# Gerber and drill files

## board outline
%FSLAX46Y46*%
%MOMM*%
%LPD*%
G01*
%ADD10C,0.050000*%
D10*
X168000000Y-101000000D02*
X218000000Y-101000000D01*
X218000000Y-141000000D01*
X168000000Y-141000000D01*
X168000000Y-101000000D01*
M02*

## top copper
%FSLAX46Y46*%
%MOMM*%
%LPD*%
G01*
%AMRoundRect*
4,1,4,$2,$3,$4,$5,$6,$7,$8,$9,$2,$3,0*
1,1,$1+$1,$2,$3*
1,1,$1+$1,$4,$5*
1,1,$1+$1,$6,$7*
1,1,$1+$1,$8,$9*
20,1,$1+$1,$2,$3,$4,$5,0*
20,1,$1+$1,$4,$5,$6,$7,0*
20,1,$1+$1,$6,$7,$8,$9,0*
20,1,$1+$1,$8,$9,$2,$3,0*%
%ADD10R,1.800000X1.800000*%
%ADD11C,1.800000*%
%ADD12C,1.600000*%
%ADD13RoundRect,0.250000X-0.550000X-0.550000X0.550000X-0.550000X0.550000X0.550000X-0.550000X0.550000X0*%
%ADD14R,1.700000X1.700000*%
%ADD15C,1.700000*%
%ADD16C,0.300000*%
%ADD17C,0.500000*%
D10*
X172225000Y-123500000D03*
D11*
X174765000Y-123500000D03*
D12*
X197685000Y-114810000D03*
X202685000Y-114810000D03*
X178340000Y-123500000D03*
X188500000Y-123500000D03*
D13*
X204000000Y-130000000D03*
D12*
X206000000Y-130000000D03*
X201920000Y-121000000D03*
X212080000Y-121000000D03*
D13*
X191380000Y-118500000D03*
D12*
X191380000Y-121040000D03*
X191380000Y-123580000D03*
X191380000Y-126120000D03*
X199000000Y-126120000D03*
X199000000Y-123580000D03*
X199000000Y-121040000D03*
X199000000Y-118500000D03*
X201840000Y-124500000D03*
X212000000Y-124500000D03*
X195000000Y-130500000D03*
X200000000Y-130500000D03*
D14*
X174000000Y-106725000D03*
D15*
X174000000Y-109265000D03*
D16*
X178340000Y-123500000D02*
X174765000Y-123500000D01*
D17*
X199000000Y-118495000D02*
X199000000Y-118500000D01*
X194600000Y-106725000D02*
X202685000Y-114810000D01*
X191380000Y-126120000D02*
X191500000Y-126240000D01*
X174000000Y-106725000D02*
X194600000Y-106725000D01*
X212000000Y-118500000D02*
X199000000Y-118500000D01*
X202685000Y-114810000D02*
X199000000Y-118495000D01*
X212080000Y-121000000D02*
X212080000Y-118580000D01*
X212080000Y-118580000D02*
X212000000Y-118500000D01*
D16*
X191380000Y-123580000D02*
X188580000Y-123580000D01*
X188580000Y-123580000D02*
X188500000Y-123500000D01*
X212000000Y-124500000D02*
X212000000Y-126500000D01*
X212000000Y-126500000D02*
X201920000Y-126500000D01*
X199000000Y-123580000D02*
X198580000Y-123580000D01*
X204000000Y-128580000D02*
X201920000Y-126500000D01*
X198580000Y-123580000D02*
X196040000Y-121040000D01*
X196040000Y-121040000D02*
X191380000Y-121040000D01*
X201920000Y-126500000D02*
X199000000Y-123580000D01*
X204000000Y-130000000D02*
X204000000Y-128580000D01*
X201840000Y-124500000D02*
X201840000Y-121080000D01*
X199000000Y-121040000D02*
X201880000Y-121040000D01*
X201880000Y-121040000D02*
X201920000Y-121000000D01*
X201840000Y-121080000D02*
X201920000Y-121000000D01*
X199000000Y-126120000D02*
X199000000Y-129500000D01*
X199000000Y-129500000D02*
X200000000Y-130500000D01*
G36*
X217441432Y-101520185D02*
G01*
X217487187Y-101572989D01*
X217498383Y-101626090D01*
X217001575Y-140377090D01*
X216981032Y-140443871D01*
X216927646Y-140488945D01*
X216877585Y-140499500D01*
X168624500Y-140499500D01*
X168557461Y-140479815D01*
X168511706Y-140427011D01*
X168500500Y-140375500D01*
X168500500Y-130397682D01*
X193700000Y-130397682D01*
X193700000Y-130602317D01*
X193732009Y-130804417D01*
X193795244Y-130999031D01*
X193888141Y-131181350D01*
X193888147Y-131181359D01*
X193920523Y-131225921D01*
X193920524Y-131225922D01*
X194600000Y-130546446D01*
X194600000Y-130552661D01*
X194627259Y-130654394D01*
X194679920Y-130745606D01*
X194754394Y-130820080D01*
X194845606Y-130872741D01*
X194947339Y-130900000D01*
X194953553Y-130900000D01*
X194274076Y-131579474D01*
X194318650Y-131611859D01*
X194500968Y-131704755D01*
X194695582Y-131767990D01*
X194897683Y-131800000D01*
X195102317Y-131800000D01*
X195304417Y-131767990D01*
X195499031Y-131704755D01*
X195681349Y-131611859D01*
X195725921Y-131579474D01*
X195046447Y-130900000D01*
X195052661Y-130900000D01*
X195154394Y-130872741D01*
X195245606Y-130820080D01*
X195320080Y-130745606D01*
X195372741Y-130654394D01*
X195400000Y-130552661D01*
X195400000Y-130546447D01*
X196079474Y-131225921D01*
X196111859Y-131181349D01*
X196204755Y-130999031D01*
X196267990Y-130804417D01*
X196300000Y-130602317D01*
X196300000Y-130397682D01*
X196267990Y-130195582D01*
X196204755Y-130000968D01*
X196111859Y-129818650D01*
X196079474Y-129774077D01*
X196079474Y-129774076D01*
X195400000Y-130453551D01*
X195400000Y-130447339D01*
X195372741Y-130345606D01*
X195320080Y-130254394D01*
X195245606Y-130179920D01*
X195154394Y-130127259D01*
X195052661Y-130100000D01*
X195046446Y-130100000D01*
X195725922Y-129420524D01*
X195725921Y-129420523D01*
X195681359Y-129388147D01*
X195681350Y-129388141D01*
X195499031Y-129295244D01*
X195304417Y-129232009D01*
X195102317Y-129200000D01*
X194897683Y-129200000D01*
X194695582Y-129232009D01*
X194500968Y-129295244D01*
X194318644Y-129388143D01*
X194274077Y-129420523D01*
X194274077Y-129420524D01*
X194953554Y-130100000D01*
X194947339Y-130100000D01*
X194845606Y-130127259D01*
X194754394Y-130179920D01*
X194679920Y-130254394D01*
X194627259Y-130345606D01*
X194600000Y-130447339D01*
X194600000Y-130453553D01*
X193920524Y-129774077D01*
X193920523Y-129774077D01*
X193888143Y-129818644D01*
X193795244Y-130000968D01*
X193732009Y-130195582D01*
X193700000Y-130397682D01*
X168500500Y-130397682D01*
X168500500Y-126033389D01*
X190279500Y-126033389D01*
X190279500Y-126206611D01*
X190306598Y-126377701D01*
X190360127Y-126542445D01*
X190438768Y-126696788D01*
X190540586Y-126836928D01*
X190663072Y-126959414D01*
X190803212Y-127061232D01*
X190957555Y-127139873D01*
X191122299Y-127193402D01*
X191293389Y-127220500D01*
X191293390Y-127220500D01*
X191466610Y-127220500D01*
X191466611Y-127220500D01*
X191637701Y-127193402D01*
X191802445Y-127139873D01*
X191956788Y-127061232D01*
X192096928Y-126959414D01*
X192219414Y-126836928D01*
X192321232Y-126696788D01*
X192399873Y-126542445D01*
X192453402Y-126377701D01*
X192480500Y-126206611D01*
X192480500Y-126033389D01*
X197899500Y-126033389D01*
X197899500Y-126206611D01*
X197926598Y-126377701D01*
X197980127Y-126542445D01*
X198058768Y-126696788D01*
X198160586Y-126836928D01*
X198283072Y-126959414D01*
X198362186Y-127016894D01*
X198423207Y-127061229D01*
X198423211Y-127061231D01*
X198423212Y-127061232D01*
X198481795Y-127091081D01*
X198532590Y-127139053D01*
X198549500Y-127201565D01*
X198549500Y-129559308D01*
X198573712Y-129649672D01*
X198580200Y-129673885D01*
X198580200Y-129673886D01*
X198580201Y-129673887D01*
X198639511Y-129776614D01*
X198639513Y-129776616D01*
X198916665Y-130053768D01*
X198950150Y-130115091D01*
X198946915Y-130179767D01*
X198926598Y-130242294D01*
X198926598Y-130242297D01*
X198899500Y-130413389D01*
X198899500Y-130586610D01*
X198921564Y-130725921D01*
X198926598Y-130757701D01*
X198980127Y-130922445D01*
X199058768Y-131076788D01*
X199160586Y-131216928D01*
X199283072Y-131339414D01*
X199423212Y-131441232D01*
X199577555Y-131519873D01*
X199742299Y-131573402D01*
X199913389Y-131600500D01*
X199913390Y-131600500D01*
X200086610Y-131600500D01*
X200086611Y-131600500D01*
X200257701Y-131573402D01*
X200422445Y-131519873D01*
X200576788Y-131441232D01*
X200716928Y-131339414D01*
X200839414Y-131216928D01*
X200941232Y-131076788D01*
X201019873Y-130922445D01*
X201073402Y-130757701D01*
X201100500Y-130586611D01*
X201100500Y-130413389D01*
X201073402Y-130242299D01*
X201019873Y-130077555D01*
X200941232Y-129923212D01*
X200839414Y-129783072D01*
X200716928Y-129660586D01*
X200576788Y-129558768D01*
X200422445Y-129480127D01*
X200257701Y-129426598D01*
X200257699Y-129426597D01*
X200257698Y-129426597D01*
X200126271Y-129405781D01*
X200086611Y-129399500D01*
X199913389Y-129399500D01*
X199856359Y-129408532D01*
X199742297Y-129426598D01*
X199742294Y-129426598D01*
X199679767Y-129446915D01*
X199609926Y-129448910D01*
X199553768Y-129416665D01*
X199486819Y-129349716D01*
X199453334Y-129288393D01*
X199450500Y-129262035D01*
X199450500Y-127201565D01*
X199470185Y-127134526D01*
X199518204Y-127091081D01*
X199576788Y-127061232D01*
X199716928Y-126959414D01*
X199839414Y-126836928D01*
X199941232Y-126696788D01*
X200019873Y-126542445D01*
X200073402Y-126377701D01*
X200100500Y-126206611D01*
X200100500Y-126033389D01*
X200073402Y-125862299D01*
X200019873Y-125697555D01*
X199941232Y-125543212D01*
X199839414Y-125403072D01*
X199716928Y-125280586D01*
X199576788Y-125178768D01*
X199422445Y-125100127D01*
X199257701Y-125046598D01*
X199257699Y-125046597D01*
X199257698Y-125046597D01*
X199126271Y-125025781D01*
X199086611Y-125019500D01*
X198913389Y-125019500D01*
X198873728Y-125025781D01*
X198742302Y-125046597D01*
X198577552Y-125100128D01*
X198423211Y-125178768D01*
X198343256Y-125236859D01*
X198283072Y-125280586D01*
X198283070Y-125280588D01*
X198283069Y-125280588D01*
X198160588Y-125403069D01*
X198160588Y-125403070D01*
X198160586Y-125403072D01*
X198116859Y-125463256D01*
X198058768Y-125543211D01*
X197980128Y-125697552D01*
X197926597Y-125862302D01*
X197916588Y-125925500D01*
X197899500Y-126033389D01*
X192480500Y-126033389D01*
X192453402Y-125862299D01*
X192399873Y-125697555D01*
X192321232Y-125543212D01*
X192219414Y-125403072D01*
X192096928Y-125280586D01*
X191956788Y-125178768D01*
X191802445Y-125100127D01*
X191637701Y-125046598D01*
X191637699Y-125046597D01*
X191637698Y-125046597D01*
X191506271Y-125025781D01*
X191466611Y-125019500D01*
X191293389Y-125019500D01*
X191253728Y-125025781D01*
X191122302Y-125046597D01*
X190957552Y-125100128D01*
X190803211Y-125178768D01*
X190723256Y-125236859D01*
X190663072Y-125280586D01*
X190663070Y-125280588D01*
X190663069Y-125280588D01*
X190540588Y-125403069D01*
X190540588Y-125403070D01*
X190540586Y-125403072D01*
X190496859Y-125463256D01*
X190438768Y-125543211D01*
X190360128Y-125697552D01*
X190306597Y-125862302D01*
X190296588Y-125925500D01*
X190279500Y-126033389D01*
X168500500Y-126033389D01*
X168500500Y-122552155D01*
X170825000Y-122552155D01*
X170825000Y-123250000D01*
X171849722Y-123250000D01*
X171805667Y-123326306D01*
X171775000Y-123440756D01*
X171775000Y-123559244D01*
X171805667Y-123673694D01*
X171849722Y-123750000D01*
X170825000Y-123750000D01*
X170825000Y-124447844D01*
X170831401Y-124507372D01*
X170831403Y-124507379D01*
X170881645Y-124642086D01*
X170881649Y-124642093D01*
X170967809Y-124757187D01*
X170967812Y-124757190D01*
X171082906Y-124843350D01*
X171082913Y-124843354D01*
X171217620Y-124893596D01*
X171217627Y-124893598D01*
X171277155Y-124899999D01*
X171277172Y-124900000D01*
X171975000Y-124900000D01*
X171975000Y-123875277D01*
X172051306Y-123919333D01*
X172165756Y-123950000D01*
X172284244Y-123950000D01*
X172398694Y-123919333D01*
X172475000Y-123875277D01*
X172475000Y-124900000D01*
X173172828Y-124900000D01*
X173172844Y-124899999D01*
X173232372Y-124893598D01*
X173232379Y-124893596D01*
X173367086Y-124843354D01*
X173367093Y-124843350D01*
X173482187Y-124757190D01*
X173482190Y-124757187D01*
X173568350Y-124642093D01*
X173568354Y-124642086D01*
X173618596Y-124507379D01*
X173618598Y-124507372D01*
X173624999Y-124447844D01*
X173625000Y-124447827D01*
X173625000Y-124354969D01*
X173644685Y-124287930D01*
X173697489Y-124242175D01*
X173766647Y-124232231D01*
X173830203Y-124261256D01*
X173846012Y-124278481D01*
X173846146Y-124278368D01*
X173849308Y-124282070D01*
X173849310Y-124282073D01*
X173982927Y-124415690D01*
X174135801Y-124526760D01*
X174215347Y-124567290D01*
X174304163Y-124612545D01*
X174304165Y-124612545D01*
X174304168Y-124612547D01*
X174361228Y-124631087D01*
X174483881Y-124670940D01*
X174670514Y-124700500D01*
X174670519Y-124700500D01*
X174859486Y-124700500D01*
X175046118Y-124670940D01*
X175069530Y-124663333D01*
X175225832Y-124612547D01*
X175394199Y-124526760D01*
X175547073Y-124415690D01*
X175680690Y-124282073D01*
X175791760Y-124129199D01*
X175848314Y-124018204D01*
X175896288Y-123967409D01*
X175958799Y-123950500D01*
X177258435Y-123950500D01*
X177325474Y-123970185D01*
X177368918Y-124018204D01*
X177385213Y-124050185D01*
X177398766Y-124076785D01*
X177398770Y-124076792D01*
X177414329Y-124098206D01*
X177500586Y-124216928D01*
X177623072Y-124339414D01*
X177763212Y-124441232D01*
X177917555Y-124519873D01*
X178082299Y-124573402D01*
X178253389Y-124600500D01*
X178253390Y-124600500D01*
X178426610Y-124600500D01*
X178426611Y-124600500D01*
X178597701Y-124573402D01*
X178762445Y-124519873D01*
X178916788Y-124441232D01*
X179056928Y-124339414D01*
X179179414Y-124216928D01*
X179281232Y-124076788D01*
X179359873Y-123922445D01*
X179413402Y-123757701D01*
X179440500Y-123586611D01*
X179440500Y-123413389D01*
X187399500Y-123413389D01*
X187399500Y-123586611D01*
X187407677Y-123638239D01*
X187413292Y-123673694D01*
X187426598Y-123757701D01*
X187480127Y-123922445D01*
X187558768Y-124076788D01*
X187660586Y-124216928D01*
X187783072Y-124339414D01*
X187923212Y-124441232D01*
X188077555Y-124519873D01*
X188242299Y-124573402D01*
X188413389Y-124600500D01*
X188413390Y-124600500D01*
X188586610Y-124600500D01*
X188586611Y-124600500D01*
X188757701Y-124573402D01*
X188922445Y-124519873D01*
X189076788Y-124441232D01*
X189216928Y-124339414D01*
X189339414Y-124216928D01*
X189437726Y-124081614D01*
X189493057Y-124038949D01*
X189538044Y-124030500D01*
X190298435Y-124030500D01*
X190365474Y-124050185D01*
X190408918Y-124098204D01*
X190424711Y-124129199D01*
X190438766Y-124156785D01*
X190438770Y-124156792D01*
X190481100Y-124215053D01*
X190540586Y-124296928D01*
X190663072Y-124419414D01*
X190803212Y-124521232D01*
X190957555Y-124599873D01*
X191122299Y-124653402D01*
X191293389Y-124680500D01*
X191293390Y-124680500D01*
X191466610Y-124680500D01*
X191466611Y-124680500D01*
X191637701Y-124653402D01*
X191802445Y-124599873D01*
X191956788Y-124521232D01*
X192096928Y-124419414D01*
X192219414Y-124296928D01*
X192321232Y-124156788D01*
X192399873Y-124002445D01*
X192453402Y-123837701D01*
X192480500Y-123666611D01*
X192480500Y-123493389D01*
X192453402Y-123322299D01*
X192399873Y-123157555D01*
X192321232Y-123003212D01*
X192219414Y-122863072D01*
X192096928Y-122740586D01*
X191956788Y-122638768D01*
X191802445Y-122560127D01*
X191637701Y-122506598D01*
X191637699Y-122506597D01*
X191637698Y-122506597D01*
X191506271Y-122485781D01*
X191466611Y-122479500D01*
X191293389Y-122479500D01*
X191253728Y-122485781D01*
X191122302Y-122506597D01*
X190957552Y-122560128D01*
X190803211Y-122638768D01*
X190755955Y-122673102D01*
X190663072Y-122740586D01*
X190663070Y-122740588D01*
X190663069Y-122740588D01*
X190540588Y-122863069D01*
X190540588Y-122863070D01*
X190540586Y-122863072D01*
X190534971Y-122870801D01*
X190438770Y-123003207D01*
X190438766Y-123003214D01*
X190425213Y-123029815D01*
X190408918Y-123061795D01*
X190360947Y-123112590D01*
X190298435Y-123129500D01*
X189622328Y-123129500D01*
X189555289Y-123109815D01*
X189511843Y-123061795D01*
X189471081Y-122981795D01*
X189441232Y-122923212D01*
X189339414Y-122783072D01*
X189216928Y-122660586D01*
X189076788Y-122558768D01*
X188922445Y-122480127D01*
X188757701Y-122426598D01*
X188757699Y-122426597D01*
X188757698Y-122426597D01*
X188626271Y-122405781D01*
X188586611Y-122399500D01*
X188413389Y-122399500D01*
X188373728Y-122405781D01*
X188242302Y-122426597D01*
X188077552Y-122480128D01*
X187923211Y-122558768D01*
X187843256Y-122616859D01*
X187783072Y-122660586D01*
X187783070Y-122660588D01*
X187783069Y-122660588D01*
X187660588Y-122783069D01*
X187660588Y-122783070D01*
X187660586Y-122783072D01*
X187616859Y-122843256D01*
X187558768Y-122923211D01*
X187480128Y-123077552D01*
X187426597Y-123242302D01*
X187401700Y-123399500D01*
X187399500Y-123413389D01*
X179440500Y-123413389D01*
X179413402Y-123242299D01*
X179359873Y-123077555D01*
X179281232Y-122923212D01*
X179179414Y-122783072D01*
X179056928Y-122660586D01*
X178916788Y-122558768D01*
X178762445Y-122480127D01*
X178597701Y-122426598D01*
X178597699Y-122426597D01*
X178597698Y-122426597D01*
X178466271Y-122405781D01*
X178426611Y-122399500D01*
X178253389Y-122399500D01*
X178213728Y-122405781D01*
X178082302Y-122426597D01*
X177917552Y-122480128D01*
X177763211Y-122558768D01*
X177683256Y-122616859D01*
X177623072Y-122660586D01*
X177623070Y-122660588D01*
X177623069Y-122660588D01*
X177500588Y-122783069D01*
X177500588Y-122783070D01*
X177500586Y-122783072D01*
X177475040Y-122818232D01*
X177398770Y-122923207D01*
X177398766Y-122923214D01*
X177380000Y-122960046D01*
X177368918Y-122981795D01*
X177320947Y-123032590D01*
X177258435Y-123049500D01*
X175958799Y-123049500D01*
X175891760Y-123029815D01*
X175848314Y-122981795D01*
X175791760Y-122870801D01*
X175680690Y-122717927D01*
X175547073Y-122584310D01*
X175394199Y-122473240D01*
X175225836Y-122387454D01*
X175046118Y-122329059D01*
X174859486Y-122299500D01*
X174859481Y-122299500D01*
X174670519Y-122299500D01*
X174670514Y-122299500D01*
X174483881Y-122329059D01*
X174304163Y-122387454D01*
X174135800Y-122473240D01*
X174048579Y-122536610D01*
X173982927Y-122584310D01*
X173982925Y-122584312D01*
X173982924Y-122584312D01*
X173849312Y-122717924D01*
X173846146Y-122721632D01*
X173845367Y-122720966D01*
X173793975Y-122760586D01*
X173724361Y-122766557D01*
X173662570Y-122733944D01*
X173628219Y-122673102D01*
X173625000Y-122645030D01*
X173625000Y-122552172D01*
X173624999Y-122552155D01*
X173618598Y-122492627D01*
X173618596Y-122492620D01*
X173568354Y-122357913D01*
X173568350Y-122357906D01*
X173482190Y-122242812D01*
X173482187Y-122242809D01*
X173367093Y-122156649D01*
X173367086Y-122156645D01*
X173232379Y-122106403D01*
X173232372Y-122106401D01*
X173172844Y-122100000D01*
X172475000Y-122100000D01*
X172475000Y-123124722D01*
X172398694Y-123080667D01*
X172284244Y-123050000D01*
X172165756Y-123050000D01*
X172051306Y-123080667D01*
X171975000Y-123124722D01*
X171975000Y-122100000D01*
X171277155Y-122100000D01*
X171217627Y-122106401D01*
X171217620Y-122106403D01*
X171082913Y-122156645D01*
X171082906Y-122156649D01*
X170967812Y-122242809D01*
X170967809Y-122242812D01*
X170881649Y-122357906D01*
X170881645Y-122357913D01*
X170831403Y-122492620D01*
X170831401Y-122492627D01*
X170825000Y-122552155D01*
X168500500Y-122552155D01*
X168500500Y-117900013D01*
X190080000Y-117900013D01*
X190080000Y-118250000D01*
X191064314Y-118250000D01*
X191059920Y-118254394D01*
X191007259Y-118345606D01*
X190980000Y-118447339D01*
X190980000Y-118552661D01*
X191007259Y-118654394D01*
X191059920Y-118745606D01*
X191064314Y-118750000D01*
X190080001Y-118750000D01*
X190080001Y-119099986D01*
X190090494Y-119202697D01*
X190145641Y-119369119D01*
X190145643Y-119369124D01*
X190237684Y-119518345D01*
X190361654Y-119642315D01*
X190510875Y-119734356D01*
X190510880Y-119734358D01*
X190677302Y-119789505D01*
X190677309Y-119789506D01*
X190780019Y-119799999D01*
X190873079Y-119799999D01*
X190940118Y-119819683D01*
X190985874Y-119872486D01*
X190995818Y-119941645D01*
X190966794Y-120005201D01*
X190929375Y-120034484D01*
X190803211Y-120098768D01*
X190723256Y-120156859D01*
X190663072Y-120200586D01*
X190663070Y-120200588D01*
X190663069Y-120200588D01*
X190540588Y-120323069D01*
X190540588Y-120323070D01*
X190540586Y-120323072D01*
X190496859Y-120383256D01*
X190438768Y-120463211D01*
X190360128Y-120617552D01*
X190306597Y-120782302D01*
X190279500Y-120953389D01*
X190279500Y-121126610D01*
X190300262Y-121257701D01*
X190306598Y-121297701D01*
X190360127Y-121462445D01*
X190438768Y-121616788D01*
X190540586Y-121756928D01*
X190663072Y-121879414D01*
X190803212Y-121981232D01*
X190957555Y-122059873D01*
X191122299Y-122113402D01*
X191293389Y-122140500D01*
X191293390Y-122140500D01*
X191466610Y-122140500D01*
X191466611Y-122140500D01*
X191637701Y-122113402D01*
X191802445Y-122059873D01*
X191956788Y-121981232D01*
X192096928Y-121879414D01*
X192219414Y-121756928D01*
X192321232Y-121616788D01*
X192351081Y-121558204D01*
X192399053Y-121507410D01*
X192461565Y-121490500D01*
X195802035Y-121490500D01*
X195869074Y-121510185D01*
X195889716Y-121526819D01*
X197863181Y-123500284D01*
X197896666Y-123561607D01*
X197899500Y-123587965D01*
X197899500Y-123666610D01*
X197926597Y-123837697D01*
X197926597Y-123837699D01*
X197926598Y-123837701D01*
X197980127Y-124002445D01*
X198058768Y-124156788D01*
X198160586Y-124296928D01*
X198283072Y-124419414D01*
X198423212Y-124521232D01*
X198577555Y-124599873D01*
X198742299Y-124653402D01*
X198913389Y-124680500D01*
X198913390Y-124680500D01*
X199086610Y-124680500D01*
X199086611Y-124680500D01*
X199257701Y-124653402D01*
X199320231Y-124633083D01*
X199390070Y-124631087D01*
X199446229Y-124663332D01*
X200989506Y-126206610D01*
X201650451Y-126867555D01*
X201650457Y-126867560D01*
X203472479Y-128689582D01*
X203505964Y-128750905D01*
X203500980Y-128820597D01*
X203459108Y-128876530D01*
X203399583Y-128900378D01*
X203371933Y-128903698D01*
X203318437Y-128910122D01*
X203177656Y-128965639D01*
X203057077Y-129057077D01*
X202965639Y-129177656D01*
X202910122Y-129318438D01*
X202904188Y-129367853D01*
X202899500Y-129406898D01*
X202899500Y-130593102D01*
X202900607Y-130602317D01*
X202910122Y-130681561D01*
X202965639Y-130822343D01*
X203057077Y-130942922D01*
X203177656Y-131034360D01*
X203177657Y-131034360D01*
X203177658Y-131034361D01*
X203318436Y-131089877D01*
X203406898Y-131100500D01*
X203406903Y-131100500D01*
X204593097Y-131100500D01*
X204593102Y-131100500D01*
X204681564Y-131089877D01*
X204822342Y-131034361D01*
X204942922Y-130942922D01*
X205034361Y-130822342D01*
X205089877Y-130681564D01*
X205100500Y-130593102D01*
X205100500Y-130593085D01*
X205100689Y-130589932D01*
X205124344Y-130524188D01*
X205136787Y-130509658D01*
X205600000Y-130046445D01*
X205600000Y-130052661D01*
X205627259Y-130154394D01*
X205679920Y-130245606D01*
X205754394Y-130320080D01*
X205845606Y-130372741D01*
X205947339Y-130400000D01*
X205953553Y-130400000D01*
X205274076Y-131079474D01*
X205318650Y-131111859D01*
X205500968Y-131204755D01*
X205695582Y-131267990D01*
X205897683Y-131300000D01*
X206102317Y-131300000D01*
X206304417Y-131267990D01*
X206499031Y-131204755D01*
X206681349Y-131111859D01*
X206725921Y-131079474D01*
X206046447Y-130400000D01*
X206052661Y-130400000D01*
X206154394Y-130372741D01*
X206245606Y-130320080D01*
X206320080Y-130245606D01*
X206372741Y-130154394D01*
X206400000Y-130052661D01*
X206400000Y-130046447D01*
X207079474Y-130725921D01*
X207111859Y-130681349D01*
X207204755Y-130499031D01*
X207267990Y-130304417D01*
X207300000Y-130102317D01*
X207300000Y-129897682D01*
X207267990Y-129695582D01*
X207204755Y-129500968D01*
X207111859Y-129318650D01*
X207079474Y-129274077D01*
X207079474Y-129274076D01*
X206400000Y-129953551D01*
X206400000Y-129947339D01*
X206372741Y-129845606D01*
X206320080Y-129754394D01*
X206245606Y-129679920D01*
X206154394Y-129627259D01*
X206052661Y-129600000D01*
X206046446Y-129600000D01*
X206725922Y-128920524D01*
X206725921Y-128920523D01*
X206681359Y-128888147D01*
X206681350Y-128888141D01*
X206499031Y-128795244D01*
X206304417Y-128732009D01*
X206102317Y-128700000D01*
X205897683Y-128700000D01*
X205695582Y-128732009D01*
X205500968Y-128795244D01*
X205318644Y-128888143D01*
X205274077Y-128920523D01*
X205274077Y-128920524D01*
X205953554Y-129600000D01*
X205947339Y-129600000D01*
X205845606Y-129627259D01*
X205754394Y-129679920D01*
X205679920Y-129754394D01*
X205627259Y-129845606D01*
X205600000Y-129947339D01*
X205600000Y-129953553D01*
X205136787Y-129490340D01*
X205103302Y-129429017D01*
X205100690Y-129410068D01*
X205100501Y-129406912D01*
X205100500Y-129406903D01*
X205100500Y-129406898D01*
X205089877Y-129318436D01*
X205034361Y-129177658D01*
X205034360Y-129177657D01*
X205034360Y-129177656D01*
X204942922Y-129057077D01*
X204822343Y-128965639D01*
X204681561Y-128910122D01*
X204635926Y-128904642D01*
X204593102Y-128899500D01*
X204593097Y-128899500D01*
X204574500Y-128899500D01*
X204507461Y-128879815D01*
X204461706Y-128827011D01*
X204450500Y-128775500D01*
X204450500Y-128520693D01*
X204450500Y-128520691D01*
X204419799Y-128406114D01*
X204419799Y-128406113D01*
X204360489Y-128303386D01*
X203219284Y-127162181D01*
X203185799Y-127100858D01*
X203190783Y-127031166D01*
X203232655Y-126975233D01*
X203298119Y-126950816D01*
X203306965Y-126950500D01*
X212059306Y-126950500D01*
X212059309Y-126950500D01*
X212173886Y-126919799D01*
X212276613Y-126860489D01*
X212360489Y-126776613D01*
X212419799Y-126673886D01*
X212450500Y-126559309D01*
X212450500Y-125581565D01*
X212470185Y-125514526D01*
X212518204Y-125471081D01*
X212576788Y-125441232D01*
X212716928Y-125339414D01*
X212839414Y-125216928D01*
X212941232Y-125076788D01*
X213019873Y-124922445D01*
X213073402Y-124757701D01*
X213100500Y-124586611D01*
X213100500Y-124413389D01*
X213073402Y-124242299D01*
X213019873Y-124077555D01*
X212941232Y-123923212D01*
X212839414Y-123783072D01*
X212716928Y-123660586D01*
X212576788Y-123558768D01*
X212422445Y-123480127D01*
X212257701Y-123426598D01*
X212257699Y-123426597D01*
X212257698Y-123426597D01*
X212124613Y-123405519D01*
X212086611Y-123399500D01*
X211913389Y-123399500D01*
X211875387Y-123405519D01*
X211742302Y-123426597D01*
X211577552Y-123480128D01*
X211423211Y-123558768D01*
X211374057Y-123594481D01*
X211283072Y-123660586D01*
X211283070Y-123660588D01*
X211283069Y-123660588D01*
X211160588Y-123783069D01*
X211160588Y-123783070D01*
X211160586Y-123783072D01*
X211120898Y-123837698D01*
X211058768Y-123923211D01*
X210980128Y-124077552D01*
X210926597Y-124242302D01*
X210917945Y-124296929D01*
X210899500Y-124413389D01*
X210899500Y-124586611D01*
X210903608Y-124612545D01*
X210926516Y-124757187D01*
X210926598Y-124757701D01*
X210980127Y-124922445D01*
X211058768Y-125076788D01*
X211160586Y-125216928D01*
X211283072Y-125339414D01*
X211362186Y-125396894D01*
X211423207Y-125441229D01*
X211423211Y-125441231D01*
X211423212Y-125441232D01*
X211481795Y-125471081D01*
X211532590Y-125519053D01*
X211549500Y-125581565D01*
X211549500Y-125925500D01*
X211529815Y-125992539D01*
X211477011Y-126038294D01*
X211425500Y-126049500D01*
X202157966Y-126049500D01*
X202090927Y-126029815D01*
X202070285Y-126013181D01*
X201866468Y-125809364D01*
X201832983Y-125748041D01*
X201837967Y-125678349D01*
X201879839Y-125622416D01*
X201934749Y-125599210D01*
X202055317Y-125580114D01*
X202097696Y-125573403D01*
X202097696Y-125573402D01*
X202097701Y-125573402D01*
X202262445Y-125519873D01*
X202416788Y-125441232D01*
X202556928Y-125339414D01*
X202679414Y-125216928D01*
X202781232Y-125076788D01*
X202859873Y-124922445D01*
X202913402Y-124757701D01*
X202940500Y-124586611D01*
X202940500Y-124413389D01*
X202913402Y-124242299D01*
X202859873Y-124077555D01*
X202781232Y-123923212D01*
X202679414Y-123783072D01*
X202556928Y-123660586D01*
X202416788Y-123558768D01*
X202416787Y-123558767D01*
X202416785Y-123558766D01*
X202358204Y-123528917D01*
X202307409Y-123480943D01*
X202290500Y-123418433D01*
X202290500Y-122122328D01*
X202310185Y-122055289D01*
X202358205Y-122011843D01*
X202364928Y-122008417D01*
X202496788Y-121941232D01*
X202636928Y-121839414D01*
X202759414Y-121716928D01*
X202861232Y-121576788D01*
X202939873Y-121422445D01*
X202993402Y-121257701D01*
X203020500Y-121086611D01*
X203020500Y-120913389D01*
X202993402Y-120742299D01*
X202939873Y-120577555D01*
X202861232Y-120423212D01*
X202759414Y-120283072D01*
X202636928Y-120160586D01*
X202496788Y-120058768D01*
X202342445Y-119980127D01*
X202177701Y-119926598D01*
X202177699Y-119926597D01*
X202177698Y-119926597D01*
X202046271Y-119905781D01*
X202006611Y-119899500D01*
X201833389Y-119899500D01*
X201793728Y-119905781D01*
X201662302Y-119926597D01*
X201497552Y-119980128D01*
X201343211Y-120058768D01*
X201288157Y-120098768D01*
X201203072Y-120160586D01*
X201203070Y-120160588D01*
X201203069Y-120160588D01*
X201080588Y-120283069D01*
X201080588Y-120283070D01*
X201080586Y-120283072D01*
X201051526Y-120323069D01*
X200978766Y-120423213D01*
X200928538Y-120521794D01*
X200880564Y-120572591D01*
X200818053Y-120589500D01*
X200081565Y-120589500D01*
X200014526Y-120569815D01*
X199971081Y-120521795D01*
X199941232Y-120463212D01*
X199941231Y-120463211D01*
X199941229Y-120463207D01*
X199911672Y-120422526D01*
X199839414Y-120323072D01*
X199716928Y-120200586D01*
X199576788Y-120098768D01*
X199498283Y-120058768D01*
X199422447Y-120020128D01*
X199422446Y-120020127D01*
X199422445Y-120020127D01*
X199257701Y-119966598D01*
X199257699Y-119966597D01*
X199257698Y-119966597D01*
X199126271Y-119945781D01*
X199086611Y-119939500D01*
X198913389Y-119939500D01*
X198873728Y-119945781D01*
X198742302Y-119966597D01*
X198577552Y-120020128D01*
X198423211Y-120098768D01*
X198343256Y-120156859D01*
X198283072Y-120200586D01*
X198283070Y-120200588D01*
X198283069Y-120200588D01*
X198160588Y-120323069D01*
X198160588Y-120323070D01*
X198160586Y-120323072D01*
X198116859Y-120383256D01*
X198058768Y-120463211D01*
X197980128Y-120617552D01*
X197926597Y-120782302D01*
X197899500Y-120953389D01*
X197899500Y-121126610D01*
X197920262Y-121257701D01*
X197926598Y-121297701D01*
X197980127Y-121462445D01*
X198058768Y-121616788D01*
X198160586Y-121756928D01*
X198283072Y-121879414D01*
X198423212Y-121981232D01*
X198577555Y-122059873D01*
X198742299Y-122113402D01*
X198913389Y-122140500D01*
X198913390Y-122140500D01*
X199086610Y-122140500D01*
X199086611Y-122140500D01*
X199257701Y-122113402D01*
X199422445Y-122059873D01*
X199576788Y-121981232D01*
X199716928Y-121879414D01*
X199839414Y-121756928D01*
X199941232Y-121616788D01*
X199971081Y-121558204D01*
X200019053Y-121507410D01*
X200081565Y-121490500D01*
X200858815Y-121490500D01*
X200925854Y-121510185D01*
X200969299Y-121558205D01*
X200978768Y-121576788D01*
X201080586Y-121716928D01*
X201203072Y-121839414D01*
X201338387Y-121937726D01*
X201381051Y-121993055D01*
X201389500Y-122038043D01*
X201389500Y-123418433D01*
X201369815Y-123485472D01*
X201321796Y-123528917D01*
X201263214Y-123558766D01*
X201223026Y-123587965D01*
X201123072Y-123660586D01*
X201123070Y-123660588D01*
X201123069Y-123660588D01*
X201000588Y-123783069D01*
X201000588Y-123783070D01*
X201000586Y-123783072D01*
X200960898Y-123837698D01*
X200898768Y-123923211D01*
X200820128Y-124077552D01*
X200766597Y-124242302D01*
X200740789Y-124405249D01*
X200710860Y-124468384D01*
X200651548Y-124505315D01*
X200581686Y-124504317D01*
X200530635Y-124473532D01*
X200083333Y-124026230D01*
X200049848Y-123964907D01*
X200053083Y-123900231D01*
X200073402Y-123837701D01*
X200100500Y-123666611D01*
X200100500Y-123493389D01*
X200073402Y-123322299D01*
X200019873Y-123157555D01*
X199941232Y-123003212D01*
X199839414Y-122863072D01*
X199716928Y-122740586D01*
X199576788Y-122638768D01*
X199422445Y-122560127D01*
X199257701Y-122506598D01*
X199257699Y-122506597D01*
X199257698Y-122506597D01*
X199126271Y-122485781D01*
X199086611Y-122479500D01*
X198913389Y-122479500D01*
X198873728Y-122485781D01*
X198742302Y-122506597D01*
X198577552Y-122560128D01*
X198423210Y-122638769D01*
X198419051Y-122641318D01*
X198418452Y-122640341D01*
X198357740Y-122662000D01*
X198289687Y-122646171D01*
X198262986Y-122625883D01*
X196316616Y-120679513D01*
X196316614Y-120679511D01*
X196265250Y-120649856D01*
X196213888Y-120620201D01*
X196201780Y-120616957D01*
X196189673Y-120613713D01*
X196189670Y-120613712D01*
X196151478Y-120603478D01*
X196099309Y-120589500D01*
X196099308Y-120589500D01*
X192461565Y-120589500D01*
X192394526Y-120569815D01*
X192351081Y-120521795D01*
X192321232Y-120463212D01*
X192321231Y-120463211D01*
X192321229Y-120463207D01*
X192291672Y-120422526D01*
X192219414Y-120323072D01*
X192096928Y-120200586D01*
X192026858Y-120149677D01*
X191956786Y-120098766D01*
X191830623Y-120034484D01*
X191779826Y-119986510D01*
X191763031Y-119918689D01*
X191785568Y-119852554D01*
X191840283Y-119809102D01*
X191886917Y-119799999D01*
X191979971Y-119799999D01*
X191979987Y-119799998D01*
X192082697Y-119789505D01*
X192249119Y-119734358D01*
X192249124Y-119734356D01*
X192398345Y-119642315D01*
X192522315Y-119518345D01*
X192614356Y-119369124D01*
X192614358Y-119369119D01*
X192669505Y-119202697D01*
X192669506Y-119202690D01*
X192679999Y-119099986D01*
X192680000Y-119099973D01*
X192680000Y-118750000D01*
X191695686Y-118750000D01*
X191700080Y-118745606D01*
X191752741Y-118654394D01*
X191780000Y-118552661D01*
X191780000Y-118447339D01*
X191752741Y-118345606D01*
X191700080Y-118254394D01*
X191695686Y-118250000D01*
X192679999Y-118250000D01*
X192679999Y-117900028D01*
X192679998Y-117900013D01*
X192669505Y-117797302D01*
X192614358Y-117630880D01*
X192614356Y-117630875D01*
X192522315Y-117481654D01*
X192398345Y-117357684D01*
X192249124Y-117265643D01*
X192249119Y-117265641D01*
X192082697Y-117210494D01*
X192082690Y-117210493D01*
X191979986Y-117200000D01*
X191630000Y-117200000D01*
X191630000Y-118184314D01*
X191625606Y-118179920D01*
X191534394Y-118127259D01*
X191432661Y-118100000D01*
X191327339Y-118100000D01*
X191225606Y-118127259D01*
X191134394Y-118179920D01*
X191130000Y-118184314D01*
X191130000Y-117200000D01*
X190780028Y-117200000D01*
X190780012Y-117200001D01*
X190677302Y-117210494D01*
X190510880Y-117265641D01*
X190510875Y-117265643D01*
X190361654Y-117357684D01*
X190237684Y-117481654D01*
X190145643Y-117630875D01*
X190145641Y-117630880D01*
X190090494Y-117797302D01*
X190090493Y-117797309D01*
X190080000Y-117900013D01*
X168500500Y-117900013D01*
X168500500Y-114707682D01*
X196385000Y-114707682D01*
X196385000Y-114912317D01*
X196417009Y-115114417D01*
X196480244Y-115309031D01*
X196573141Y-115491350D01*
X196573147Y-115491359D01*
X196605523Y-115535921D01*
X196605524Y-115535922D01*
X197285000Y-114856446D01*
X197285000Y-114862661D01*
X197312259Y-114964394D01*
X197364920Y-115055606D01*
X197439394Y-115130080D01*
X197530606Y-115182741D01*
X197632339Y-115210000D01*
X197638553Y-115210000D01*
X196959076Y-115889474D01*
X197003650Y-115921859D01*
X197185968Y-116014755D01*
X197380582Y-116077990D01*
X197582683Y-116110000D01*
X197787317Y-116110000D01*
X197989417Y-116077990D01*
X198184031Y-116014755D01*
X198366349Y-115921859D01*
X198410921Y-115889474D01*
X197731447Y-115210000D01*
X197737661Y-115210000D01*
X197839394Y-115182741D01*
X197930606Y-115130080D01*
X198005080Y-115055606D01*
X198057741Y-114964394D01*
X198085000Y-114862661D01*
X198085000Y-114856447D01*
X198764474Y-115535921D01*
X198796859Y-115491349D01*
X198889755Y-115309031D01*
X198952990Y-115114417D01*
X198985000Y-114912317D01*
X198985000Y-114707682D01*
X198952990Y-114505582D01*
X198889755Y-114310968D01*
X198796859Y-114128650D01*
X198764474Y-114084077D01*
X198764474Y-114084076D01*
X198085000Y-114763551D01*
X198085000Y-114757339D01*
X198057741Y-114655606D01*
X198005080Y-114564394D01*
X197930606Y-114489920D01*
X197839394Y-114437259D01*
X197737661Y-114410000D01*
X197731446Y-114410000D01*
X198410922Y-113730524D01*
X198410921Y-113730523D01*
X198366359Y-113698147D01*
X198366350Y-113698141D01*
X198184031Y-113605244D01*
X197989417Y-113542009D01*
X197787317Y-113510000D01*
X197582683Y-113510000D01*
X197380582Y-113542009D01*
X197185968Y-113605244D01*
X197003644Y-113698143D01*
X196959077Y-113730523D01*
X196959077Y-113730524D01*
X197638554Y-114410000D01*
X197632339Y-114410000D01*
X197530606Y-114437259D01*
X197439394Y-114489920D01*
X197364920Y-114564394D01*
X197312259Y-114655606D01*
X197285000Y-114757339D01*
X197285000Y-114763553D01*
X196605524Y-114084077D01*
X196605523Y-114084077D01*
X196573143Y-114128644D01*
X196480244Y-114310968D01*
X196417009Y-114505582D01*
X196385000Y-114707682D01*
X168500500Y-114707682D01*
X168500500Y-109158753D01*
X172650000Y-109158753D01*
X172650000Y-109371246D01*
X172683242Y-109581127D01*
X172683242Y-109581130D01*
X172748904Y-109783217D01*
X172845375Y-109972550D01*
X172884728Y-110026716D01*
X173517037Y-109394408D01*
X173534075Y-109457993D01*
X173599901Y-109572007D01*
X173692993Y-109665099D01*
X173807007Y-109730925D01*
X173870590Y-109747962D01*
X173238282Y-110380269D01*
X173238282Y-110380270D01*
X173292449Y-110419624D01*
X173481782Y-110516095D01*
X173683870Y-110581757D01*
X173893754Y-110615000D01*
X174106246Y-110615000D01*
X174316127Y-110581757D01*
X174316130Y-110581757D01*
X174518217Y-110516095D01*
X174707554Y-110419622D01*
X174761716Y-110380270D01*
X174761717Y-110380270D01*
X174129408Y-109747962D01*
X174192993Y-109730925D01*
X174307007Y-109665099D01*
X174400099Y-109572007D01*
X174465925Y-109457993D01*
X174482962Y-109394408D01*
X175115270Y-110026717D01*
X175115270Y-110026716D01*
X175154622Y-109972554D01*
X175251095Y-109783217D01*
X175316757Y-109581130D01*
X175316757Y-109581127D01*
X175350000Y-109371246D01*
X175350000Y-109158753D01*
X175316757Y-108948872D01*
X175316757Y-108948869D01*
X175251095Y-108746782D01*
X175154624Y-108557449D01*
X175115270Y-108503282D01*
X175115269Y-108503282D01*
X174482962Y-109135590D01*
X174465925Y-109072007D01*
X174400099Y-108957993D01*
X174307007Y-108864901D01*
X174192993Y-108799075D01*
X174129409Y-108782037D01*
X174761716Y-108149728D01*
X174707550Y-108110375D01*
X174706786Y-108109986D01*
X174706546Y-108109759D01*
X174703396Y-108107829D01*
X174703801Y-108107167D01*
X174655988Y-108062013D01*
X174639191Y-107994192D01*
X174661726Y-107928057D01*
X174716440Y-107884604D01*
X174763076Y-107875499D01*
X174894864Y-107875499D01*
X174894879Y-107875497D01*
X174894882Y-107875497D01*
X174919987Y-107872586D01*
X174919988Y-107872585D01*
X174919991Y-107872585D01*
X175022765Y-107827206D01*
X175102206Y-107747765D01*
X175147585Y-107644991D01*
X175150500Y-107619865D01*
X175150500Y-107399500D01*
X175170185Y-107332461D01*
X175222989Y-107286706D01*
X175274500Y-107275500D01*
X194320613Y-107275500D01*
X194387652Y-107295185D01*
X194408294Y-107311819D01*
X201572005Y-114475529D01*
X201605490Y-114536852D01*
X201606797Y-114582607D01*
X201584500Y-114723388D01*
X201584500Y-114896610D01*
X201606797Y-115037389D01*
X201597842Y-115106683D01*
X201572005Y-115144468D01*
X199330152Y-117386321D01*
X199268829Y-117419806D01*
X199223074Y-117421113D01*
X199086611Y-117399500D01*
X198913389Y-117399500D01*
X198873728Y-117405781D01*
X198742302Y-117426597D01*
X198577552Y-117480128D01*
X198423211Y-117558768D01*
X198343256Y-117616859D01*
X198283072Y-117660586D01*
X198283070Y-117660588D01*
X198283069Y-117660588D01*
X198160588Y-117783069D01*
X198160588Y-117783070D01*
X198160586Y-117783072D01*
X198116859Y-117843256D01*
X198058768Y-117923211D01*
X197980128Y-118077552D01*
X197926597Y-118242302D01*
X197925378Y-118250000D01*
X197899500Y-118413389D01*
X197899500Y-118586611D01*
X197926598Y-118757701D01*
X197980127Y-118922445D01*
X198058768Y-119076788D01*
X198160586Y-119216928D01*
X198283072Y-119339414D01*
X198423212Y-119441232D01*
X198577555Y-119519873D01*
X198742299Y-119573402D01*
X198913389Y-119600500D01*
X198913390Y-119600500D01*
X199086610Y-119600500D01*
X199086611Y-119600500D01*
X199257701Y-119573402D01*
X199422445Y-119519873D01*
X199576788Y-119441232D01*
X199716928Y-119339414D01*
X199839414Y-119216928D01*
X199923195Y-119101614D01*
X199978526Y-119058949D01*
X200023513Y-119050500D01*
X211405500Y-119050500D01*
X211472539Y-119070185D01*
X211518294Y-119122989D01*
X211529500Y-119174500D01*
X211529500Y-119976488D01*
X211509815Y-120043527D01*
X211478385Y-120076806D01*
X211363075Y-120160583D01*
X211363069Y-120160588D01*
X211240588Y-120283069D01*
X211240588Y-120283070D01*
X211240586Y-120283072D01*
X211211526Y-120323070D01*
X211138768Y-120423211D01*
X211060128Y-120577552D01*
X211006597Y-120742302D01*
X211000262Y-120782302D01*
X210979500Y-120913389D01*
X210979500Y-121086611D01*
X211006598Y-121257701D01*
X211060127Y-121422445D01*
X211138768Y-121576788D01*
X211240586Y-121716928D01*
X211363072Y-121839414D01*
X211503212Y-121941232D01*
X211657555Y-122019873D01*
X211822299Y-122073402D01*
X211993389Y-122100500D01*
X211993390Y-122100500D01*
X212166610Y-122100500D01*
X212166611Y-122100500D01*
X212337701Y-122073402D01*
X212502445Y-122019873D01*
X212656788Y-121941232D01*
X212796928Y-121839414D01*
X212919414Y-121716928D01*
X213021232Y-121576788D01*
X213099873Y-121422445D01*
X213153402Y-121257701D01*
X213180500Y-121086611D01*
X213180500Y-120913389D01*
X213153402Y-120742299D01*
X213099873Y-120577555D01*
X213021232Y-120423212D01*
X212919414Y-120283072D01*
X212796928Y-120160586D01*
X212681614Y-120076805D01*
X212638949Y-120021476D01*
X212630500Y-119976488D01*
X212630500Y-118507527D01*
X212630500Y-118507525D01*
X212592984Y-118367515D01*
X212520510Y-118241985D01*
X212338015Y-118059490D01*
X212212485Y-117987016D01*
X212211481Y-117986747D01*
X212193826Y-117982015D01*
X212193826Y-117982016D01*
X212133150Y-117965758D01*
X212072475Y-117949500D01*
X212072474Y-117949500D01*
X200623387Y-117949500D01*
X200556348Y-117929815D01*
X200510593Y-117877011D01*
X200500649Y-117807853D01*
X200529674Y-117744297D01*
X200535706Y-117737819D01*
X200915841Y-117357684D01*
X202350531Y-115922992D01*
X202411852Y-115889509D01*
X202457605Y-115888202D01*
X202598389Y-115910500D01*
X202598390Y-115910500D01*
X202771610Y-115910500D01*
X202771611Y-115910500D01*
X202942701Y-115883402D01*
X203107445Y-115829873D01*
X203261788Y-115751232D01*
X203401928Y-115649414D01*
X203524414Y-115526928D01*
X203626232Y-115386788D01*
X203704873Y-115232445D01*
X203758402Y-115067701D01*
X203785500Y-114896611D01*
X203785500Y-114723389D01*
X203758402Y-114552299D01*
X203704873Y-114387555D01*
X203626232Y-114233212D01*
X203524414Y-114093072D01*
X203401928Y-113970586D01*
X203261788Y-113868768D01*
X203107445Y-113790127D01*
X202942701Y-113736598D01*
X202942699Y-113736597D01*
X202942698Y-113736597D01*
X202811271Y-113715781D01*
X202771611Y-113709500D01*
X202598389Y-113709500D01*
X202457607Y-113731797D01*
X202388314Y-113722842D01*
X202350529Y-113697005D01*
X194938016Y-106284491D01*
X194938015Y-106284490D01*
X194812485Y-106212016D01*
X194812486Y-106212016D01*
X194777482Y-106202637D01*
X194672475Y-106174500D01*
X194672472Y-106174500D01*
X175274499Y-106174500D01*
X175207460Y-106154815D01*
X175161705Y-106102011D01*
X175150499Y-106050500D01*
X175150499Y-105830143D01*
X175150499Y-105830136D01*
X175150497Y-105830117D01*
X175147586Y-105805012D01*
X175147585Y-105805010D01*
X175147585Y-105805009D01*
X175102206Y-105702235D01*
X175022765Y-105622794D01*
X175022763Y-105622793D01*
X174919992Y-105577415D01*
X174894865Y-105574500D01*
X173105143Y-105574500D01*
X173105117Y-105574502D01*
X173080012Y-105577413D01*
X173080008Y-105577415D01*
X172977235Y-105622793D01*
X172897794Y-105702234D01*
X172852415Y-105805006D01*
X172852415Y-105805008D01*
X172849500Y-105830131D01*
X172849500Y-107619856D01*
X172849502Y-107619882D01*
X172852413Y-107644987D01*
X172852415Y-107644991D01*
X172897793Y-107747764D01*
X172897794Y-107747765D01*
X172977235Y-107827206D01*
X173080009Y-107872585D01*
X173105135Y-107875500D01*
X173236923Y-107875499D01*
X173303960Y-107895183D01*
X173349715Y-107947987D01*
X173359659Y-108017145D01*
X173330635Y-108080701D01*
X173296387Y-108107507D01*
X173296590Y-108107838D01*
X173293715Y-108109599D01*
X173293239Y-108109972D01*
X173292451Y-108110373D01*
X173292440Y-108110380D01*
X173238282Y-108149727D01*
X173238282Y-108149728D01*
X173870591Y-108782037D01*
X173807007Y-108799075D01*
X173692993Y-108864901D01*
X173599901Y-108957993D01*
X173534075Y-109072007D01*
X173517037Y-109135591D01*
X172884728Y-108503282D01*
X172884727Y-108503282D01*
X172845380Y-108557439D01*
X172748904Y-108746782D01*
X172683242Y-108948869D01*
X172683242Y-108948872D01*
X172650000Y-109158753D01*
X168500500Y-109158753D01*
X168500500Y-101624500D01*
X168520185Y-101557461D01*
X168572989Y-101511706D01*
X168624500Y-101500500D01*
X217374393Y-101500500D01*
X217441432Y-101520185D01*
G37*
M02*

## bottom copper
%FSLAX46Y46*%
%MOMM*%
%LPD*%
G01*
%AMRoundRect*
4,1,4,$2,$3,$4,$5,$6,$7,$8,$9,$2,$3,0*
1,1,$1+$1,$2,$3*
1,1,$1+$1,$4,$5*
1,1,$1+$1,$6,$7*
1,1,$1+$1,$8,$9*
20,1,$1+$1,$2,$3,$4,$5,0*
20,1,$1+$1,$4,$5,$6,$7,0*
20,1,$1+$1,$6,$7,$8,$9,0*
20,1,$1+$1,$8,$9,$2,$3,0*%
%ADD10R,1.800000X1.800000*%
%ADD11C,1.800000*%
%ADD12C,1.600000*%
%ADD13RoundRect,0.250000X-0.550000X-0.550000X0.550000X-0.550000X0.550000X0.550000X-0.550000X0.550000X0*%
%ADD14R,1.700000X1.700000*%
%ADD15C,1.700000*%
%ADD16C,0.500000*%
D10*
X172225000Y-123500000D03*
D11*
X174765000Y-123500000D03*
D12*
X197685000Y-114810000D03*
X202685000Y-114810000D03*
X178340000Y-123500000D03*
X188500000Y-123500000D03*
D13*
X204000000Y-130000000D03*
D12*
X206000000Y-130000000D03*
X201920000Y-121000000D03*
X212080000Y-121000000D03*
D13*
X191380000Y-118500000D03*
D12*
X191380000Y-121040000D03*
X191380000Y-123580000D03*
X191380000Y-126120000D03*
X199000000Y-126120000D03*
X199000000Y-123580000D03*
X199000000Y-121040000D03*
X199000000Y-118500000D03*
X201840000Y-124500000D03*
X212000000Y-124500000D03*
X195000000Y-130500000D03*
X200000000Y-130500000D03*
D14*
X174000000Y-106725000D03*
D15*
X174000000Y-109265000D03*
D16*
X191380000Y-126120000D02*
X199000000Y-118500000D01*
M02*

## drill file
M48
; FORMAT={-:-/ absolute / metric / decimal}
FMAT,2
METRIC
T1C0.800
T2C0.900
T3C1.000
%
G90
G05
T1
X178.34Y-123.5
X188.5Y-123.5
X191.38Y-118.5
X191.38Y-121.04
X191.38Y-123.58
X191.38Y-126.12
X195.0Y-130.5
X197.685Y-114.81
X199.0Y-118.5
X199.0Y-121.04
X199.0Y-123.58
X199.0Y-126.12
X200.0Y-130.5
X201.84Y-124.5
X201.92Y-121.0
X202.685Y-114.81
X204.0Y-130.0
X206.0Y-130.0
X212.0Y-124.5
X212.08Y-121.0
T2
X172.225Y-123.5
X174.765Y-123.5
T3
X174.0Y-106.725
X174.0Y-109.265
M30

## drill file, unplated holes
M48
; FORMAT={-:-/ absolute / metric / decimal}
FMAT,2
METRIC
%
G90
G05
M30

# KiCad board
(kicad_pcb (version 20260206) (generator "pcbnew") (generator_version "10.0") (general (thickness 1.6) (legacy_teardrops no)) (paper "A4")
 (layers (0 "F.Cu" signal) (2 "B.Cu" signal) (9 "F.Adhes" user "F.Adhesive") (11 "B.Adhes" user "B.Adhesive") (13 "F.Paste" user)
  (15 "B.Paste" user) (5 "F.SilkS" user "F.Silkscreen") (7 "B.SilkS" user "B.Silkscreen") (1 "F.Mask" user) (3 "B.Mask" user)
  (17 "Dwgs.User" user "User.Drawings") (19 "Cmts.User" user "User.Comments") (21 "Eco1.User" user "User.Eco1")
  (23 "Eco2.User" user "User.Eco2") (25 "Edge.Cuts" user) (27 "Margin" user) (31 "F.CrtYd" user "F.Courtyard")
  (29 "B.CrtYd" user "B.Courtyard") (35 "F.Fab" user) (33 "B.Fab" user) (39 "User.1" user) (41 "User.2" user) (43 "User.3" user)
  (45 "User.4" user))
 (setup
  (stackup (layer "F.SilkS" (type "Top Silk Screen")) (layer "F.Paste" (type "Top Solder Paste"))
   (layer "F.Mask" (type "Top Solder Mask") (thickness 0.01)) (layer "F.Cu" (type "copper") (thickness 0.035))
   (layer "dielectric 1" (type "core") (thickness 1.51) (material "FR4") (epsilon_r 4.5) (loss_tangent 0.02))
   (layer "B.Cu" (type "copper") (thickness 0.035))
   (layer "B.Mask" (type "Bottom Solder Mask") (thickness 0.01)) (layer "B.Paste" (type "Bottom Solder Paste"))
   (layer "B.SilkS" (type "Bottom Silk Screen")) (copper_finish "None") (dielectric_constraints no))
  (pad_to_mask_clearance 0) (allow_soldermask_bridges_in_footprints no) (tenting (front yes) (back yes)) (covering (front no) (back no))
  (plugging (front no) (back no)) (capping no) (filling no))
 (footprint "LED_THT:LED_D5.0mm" (layer "F.Cu") (at 172.225 123.5)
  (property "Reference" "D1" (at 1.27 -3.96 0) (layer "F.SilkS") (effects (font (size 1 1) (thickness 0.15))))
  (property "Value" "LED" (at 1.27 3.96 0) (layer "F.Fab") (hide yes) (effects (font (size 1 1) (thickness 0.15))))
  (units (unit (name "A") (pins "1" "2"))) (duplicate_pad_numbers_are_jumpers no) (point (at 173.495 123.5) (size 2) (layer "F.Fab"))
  (pad "1" thru_hole rect (at 0 0) (size 1.8 1.8) (drill 0.9) (layers "*.Cu" "*.Mask") (remove_unused_layers no) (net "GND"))
  (pad "2" thru_hole circle (at 2.54 0) (size 1.8 1.8) (drill 0.9) (layers "*.Cu" "*.Mask") (remove_unused_layers no) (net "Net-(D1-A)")))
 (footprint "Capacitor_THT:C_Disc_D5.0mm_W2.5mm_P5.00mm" (layer "F.Cu") (at 197.685 114.81)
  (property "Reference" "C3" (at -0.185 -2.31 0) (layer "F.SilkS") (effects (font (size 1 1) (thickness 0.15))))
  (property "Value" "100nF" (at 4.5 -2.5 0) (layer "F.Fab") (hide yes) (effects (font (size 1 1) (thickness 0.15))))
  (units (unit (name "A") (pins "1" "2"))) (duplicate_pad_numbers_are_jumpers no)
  (pad "1" thru_hole circle (at 0 0) (size 1.6 1.6) (drill 0.8) (layers "*.Cu" "*.Mask") (remove_unused_layers no) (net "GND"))
  (pad "2" thru_hole circle (at 5 0) (size 1.6 1.6) (drill 0.8) (layers "*.Cu" "*.Mask") (remove_unused_layers no) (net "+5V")))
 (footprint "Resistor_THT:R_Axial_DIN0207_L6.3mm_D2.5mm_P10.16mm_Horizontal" (layer "F.Cu") (at 178.34 123.5)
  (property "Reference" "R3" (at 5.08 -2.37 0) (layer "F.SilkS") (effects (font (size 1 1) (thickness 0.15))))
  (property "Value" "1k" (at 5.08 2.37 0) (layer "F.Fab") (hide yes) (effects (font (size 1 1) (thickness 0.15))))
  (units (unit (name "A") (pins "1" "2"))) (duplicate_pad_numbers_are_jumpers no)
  (pad "1" thru_hole circle (at 0 0) (size 1.6 1.6) (drill 0.8) (layers "*.Cu" "*.Mask") (remove_unused_layers no) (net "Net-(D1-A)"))
  (pad "2" thru_hole circle (at 10.16 0) (size 1.6 1.6) (drill 0.8) (layers "*.Cu" "*.Mask") (remove_unused_layers no) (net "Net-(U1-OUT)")))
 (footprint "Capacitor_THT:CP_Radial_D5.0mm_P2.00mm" (layer "F.Cu") (at 204 130)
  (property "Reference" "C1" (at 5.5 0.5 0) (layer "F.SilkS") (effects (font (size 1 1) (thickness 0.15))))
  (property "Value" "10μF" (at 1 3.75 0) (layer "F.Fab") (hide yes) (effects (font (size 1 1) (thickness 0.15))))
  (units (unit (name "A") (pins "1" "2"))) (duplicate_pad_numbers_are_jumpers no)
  (pad "1" thru_hole roundrect (at 0 0) (size 1.6 1.6) (drill 0.8) (layers "*.Cu" "*.Mask") (remove_unused_layers no)
   (roundrect_rratio 0.15625) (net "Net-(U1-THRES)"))
  (pad "2" thru_hole circle (at 2 0) (size 1.6 1.6) (drill 0.8) (layers "*.Cu" "*.Mask") (remove_unused_layers no) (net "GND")))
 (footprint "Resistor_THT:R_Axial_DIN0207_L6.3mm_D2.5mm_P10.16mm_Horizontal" (layer "F.Cu") (at 201.92 121)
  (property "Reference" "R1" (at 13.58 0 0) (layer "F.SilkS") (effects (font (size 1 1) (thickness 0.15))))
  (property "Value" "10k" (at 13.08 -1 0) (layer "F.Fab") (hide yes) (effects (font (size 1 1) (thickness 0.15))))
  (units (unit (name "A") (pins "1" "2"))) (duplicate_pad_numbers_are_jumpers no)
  (pad "1" thru_hole circle (at 0 0) (size 1.6 1.6) (drill 0.8) (layers "*.Cu" "*.Mask") (remove_unused_layers no) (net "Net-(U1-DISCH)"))
  (pad "2" thru_hole circle (at 10.16 0) (size 1.6 1.6) (drill 0.8) (layers "*.Cu" "*.Mask") (remove_unused_layers no) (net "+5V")))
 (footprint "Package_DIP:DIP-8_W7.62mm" (layer "F.Cu") (at 191.38 118.5)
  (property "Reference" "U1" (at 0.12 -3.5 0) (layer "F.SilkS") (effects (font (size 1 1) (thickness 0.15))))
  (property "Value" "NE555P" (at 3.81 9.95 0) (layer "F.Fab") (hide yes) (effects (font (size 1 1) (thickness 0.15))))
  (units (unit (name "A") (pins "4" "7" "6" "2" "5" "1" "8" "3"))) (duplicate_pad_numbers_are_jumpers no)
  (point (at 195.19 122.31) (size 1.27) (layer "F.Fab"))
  (pad "1" thru_hole roundrect (at 0 0) (size 1.6 1.6) (drill 0.8) (layers "*.Cu" "*.Mask") (remove_unused_layers no)
   (roundrect_rratio 0.15625) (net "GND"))
  (pad "2" thru_hole circle (at 0 2.54) (size 1.6 1.6) (drill 0.8) (layers "*.Cu" "*.Mask") (remove_unused_layers no) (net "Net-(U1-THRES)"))
  (pad "3" thru_hole circle (at 0 5.08) (size 1.6 1.6) (drill 0.8) (layers "*.Cu" "*.Mask") (remove_unused_layers no) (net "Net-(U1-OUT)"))
  (pad "4" thru_hole circle (at 0 7.62) (size 1.6 1.6) (drill 0.8) (layers "*.Cu" "*.Mask") (remove_unused_layers no) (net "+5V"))
  (pad "5" thru_hole circle (at 7.62 7.62) (size 1.6 1.6) (drill 0.8) (layers "*.Cu" "*.Mask") (remove_unused_layers no)
   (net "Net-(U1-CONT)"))
  (pad "6" thru_hole circle (at 7.62 5.08) (size 1.6 1.6) (drill 0.8) (layers "*.Cu" "*.Mask") (remove_unused_layers no)
   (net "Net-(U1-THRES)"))
  (pad "7" thru_hole circle (at 7.62 2.54) (size 1.6 1.6) (drill 0.8) (layers "*.Cu" "*.Mask") (remove_unused_layers no)
   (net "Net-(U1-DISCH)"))
  (pad "8" thru_hole circle (at 7.62 0) (size 1.6 1.6) (drill 0.8) (layers "*.Cu" "*.Mask") (remove_unused_layers no) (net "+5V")))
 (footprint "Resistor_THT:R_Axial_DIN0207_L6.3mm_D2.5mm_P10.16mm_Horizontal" (layer "F.Cu") (at 201.84 124.5)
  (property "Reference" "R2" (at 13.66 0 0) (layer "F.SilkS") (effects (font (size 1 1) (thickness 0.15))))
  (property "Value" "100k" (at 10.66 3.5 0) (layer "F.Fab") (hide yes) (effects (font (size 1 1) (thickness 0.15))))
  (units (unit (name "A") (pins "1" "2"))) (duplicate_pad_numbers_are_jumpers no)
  (pad "1" thru_hole circle (at 0 0) (size 1.6 1.6) (drill 0.8) (layers "*.Cu" "*.Mask") (remove_unused_layers no) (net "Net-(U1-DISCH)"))
  (pad "2" thru_hole circle (at 10.16 0) (size 1.6 1.6) (drill 0.8) (layers "*.Cu" "*.Mask") (remove_unused_layers no)
   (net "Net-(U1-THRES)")))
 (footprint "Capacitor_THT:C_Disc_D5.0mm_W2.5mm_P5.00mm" (layer "F.Cu") (at 195 130.5)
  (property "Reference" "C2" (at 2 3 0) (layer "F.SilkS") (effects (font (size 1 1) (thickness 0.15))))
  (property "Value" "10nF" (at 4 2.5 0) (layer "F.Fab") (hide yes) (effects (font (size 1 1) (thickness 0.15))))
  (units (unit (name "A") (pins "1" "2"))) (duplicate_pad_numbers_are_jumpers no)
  (pad "1" thru_hole circle (at 0 0) (size 1.6 1.6) (drill 0.8) (layers "*.Cu" "*.Mask") (remove_unused_layers no) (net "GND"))
  (pad "2" thru_hole circle (at 5 0) (size 1.6 1.6) (drill 0.8) (layers "*.Cu" "*.Mask") (remove_unused_layers no) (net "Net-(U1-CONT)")))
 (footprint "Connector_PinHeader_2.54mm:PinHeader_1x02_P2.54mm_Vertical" (layer "F.Cu") (at 174 106.725)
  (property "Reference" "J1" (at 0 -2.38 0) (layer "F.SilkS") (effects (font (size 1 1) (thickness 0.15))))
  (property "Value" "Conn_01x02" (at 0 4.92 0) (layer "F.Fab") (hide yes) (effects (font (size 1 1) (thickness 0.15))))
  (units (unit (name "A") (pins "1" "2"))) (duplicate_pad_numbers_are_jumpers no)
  (pad "1" thru_hole rect (at 0 0) (size 1.7 1.7) (drill 1) (layers "*.Cu" "*.Mask") (remove_unused_layers no) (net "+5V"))
  (pad "2" thru_hole circle (at 0 2.54) (size 1.7 1.7) (drill 1) (layers "*.Cu" "*.Mask") (remove_unused_layers no) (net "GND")))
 (gr_rect (start 168 101) (end 218 141) (stroke (width 0.05) (type default)) (fill no) (layer "Edge.Cuts"))
 (segment (start 178.34 123.5) (end 174.765 123.5) (width 0.3) (layer "F.Cu") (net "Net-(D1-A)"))
 (segment (start 199 118.495) (end 199 118.5) (width 0.5) (layer "F.Cu") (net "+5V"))
 (segment (start 194.6 106.725) (end 202.685 114.81) (width 0.5) (layer "F.Cu") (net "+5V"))
 (segment (start 191.38 126.12) (end 191.5 126.24) (width 0.5) (layer "F.Cu") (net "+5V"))
 (segment (start 174 106.725) (end 194.6 106.725) (width 0.5) (layer "F.Cu") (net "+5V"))
 (segment (start 212 118.5) (end 199 118.5) (width 0.5) (layer "F.Cu") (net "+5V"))
 (segment (start 202.685 114.81) (end 199 118.495) (width 0.5) (layer "F.Cu") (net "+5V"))
 (segment (start 212.08 121) (end 212.08 118.58) (width 0.5) (layer "F.Cu") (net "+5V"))
 (segment (start 212.08 118.58) (end 212 118.5) (width 0.5) (layer "F.Cu") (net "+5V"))
 (segment (start 191.38 126.12) (end 199 118.5) (width 0.5) (layer "B.Cu") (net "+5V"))
 (segment (start 191.38 123.58) (end 188.58 123.58) (width 0.3) (layer "F.Cu") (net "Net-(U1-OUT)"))
 (segment (start 188.58 123.58) (end 188.5 123.5) (width 0.3) (layer "F.Cu") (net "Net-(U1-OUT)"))
 (segment (start 212 124.5) (end 212 126.5) (width 0.3) (layer "F.Cu") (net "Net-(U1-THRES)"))
 (segment (start 212 126.5) (end 201.92 126.5) (width 0.3) (layer "F.Cu") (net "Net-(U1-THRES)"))
 (segment (start 199 123.58) (end 198.58 123.58) (width 0.3) (layer "F.Cu") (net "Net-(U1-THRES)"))
 (segment (start 204 128.58) (end 201.92 126.5) (width 0.3) (layer "F.Cu") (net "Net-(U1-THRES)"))
 (segment (start 198.58 123.58) (end 196.04 121.04) (width 0.3) (layer "F.Cu") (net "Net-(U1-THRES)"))
 (segment (start 196.04 121.04) (end 191.38 121.04) (width 0.3) (layer "F.Cu") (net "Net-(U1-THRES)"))
 (segment (start 201.92 126.5) (end 199 123.58) (width 0.3) (layer "F.Cu") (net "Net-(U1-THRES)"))
 (segment (start 204 130) (end 204 128.58) (width 0.3) (layer "F.Cu") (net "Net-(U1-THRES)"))
 (segment (start 201.84 124.5) (end 201.84 121.08) (width 0.3) (layer "F.Cu") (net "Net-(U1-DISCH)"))
 (segment (start 199 121.04) (end 201.88 121.04) (width 0.3) (layer "F.Cu") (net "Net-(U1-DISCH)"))
 (segment (start 201.88 121.04) (end 201.92 121) (width 0.3) (layer "F.Cu") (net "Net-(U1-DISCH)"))
 (segment (start 201.84 121.08) (end 201.92 121) (width 0.3) (layer "F.Cu") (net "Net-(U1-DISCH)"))
 (segment (start 199 126.12) (end 199 129.5) (width 0.3) (layer "F.Cu") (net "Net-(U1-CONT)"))
 (segment (start 199 129.5) (end 200 130.5) (width 0.3) (layer "F.Cu") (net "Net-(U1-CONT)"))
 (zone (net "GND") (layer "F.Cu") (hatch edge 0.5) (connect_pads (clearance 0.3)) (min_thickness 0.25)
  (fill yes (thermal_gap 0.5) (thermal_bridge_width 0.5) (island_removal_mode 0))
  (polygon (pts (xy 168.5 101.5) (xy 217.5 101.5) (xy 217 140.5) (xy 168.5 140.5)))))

